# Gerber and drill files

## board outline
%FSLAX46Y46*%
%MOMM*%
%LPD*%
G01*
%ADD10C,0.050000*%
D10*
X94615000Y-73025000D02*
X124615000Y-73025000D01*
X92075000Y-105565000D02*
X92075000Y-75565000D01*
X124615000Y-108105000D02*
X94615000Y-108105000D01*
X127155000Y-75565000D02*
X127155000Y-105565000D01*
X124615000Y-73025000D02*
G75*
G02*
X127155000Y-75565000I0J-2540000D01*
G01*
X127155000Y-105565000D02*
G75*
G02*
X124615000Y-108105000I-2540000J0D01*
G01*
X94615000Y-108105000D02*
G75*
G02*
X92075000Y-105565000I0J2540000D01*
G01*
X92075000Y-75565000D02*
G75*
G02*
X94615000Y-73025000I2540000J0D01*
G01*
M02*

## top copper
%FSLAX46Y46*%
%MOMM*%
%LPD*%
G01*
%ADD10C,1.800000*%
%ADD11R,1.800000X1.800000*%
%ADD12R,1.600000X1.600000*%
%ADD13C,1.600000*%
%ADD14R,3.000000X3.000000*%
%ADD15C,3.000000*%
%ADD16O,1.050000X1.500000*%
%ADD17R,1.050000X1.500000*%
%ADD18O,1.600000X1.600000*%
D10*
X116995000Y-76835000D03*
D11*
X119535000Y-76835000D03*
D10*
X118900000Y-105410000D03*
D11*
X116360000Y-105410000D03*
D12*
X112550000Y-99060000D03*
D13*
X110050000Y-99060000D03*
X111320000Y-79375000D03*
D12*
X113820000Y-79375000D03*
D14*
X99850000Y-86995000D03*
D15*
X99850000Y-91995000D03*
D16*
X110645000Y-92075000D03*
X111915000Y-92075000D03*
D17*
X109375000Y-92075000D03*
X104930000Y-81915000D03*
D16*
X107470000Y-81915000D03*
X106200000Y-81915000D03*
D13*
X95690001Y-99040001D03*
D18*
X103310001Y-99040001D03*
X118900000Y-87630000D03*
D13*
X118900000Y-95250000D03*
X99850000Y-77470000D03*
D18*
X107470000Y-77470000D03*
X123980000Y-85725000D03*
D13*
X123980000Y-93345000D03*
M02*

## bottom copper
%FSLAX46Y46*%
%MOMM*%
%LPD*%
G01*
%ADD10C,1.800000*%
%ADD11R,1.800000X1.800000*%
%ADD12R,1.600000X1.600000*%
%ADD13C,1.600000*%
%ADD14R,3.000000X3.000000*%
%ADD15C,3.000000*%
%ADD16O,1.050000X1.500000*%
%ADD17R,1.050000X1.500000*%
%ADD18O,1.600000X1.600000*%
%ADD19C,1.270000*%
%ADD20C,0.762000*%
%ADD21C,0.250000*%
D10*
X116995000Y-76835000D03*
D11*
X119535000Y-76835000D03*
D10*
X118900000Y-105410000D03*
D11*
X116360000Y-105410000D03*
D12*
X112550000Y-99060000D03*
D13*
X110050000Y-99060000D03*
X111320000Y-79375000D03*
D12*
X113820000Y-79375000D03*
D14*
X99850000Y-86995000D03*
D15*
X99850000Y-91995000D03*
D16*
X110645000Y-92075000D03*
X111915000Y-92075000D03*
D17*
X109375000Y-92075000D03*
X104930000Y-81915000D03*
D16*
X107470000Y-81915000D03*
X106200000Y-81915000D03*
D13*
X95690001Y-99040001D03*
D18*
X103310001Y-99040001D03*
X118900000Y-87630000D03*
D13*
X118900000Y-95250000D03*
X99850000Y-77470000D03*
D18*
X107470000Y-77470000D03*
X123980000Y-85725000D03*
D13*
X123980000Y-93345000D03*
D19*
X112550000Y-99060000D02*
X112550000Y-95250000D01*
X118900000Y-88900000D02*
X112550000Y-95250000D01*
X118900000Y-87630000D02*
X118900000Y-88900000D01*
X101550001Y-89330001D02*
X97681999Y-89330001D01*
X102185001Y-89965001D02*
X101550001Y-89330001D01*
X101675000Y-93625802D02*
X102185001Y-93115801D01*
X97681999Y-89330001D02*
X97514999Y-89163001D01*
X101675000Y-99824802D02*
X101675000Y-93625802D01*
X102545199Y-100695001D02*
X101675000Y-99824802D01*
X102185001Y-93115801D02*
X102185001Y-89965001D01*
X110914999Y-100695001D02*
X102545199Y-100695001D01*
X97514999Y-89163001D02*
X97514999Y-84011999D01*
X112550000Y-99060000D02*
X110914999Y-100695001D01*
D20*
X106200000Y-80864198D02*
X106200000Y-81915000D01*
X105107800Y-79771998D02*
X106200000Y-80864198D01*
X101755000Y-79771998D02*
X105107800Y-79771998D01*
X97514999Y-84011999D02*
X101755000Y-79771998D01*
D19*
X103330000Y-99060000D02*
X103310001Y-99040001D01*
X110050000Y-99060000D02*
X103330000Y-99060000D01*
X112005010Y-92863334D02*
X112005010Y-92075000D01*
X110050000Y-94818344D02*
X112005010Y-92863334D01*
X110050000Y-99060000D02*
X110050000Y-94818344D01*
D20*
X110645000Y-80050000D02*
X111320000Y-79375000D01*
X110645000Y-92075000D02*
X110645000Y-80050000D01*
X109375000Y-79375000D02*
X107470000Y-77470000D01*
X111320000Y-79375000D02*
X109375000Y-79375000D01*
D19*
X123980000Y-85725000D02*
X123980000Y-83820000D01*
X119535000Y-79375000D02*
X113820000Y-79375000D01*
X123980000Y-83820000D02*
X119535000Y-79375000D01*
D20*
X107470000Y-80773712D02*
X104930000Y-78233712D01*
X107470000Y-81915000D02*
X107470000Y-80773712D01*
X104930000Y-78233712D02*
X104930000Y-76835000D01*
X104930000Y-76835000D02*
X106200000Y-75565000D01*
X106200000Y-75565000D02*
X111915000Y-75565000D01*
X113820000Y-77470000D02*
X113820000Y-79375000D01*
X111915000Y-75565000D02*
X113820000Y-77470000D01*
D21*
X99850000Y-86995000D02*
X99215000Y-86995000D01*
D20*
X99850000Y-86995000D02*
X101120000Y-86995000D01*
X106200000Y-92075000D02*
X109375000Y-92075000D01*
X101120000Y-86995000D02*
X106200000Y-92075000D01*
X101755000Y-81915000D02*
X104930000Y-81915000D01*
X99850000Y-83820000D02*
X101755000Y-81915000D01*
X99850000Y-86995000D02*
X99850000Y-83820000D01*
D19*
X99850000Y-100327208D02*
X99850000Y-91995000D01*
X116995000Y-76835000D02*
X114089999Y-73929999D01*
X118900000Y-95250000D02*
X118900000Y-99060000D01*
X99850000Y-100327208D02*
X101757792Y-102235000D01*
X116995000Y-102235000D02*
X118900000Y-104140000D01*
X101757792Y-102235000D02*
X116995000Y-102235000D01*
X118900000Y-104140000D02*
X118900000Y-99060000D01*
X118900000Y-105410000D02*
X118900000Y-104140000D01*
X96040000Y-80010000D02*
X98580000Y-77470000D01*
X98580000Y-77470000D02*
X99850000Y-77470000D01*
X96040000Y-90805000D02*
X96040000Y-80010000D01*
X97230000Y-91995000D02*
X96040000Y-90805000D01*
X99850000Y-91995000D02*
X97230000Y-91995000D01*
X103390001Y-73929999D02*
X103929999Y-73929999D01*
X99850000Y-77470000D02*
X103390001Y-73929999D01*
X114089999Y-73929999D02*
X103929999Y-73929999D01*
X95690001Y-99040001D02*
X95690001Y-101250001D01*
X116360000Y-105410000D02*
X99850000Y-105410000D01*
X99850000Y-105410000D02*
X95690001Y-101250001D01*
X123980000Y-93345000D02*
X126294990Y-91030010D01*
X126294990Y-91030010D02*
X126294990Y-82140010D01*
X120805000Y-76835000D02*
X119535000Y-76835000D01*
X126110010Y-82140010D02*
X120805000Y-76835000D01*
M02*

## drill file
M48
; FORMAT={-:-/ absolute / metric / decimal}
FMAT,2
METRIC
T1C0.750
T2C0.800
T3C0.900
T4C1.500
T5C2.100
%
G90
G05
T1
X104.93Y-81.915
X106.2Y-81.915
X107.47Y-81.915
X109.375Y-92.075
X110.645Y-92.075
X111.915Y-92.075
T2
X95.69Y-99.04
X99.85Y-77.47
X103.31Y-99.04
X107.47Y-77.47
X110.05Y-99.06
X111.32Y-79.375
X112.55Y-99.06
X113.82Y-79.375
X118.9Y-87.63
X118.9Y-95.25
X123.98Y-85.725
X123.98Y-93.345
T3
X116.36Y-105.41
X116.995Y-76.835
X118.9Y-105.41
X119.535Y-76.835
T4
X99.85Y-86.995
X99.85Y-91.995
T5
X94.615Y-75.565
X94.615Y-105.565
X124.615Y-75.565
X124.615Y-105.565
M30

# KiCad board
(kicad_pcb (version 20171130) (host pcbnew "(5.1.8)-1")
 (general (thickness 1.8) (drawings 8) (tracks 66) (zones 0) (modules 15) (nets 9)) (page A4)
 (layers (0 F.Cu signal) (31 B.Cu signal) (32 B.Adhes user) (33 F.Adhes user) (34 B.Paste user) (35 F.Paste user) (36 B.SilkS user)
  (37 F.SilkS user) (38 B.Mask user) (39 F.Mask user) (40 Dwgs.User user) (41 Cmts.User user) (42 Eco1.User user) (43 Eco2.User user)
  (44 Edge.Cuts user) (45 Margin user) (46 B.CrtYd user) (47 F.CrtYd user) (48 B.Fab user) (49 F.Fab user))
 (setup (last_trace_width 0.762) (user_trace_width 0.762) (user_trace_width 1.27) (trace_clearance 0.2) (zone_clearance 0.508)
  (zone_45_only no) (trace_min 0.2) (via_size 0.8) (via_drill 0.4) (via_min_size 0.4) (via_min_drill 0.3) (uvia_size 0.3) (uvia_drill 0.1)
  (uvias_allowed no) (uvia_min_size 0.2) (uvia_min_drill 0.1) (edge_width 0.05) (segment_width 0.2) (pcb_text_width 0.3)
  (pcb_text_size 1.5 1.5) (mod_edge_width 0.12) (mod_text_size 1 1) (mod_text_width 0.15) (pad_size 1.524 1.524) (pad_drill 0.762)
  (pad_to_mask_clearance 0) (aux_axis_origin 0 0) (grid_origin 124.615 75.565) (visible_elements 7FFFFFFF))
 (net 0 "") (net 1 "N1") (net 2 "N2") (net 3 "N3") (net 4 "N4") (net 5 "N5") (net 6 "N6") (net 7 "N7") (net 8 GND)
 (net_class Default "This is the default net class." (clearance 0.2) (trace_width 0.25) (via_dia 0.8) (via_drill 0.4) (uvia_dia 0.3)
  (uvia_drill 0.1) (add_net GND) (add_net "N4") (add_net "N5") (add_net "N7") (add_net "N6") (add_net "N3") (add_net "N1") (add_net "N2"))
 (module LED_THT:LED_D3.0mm (layer F.Cu) (at 119.535 76.835 180)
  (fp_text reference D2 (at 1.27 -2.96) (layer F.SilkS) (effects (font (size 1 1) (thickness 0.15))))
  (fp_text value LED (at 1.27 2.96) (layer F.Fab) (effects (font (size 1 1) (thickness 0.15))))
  (pad 2 thru_hole circle (at 2.54 0 180) (size 1.8 1.8) (drill 0.9) (layers *.Cu *.Mask) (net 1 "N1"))
  (pad 1 thru_hole rect (at 0 0 180) (size 1.8 1.8) (drill 0.9) (layers *.Cu *.Mask) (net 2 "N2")))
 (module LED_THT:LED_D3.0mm (layer F.Cu) (at 116.36 105.41)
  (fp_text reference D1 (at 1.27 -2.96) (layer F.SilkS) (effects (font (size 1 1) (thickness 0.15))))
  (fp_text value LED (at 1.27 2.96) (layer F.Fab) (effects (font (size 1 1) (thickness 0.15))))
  (pad 2 thru_hole circle (at 2.54 0) (size 1.8 1.8) (drill 0.9) (layers *.Cu *.Mask) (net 1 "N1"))
  (pad 1 thru_hole rect (at 0 0) (size 1.8 1.8) (drill 0.9) (layers *.Cu *.Mask) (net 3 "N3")))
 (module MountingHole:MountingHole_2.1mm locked (layer F.Cu) (at 124.615 105.565)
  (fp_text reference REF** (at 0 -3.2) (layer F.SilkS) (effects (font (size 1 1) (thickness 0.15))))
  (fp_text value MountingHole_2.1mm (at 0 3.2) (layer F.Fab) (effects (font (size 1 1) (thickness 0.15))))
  (pad "" np_thru_hole circle (at 0 0) (size 2.1 2.1) (drill 2.1) (layers *.Cu *.Mask)))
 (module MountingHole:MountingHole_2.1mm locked (layer F.Cu) (at 94.615 105.565)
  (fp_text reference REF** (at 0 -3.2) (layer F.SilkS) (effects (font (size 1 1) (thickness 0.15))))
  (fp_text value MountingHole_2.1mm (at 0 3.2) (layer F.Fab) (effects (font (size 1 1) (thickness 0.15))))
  (pad "" np_thru_hole circle (at 0 0) (size 2.1 2.1) (drill 2.1) (layers *.Cu *.Mask)))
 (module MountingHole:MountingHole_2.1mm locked (layer F.Cu) (at 124.615 75.565)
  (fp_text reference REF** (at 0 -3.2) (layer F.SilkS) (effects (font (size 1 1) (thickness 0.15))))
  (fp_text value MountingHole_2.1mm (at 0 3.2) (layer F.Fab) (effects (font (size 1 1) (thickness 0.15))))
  (pad "" np_thru_hole circle (at 0 0) (size 2.1 2.1) (drill 2.1) (layers *.Cu *.Mask)))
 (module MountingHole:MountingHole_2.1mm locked (layer F.Cu) (at 94.615 75.565)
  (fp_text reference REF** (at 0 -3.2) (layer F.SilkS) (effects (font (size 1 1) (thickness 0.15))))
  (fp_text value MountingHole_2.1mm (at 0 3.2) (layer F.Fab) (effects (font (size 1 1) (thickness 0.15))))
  (pad "" np_thru_hole circle (at 0 0) (size 2.1 2.1) (drill 2.1) (layers *.Cu *.Mask)))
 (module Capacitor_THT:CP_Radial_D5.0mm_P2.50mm (layer F.Cu) (at 112.55 99.06 180)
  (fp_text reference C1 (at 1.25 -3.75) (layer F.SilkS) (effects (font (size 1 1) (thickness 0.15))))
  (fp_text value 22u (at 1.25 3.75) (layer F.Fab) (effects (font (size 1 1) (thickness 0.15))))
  (pad 1 thru_hole rect (at 0 0 180) (size 1.6 1.6) (drill 0.8) (layers *.Cu *.Mask) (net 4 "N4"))
  (pad 2 thru_hole circle (at 2.5 0 180) (size 1.6 1.6) (drill 0.8) (layers *.Cu *.Mask) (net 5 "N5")))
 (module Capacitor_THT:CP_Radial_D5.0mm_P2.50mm (layer F.Cu) (at 113.82 79.375 180)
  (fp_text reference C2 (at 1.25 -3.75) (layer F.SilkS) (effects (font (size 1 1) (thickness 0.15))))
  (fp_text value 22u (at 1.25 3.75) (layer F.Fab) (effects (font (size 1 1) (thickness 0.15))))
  (pad 2 thru_hole circle (at 2.5 0 180) (size 1.6 1.6) (drill 0.8) (layers *.Cu *.Mask) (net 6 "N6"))
  (pad 1 thru_hole rect (at 0 0 180) (size 1.6 1.6) (drill 0.8) (layers *.Cu *.Mask) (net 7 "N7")))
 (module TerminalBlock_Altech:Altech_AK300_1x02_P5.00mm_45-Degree (layer F.Cu) (at 99.85 86.995 270)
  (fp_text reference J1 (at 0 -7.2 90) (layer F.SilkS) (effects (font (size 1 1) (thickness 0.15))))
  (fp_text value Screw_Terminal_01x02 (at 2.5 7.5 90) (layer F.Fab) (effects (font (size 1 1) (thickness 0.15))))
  (pad 1 thru_hole rect (at 0 0 270) (size 3 3) (drill 1.5) (layers *.Cu *.Mask) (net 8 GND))
  (pad 2 thru_hole circle (at 5 0 270) (size 3 3) (drill 1.5) (layers *.Cu *.Mask) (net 1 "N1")))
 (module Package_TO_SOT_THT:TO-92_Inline (layer F.Cu) (at 109.375 92.075)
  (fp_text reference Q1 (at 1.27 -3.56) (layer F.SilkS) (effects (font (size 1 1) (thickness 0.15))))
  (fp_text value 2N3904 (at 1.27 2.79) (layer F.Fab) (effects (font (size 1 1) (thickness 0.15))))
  (pad 2 thru_hole oval (at 1.27 0) (size 1.05 1.5) (drill 0.75) (layers *.Cu *.Mask) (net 6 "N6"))
  (pad 3 thru_hole oval (at 2.54 0) (size 1.05 1.5) (drill 0.75) (layers *.Cu *.Mask) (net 5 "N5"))
  (pad 1 thru_hole rect (at 0 0) (size 1.05 1.5) (drill 0.75) (layers *.Cu *.Mask) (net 8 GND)))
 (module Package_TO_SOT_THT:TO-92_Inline (layer F.Cu) (at 104.93 81.915)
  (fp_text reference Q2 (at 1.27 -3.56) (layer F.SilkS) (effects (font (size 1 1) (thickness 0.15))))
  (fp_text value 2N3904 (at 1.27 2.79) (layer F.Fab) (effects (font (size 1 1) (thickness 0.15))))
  (pad 1 thru_hole rect (at 0 0) (size 1.05 1.5) (drill 0.75) (layers *.Cu *.Mask) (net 8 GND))
  (pad 3 thru_hole oval (at 2.54 0) (size 1.05 1.5) (drill 0.75) (layers *.Cu *.Mask) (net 7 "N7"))
  (pad 2 thru_hole oval (at 1.27 0) (size 1.05 1.5) (drill 0.75) (layers *.Cu *.Mask) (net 4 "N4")))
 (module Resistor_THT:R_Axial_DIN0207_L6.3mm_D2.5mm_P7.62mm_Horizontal (layer F.Cu) (at 95.690001 99.040001)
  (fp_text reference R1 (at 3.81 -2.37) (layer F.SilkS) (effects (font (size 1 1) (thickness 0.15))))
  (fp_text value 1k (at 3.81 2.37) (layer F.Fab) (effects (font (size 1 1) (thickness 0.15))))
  (pad 1 thru_hole circle (at 0 0) (size 1.6 1.6) (drill 0.8) (layers *.Cu *.Mask) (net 3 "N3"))
  (pad 2 thru_hole oval (at 7.62 0) (size 1.6 1.6) (drill 0.8) (layers *.Cu *.Mask) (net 5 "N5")))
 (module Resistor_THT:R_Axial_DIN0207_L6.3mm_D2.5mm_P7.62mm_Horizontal (layer F.Cu) (at 118.9 95.25 90)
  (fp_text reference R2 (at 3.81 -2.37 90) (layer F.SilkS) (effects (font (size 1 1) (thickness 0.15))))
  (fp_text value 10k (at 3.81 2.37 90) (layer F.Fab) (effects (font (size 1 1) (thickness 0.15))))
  (pad 2 thru_hole oval (at 7.62 0 90) (size 1.6 1.6) (drill 0.8) (layers *.Cu *.Mask) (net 4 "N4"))
  (pad 1 thru_hole circle (at 0 0 90) (size 1.6 1.6) (drill 0.8) (layers *.Cu *.Mask) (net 1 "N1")))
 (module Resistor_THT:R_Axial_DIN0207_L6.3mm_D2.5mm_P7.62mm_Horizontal (layer F.Cu) (at 99.85 77.47)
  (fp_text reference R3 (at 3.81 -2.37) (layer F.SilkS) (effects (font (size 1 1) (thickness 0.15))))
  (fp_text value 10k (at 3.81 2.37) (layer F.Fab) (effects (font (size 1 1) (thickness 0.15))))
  (pad 1 thru_hole circle (at 0 0) (size 1.6 1.6) (drill 0.8) (layers *.Cu *.Mask) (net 1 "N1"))
  (pad 2 thru_hole oval (at 7.62 0) (size 1.6 1.6) (drill 0.8) (layers *.Cu *.Mask) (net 6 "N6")))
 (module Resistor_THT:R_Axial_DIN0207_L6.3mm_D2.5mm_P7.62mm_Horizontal (layer F.Cu) (at 123.98 93.345 90)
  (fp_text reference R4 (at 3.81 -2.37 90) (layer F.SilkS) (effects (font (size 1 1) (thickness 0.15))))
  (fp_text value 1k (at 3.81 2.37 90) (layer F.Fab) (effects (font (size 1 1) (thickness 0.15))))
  (pad 2 thru_hole oval (at 7.62 0 90) (size 1.6 1.6) (drill 0.8) (layers *.Cu *.Mask) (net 7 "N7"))
  (pad 1 thru_hole circle (at 0 0 90) (size 1.6 1.6) (drill 0.8) (layers *.Cu *.Mask) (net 2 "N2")))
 (gr_line (start 94.615 73.025) (end 124.615 73.025) (layer Edge.Cuts) (width 0.05))
 (gr_line (start 92.075 105.565) (end 92.075 75.565) (layer Edge.Cuts) (width 0.05))
 (gr_line (start 124.615 108.105) (end 94.615 108.105) (layer Edge.Cuts) (width 0.05))
 (gr_line (start 127.155 75.565) (end 127.155 105.565) (layer Edge.Cuts) (width 0.05))
 (gr_arc (start 124.615 75.565) (end 127.155 75.565) (angle -90) (layer Edge.Cuts) (width 0.05))
 (gr_arc (start 124.615 105.565) (end 124.615 108.105) (angle -90) (layer Edge.Cuts) (width 0.05))
 (gr_arc (start 94.615 105.565) (end 92.075 105.565) (angle -90) (layer Edge.Cuts) (width 0.05))
 (gr_arc (start 94.615 75.565) (end 94.615 73.025) (angle -90) (layer Edge.Cuts) (width 0.05))
 (segment (start 112.55 99.06) (end 112.55 95.25) (width 1.27) (layer B.Cu) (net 4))
 (segment (start 118.9 88.9) (end 112.55 95.25) (width 1.27) (layer B.Cu) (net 4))
 (segment (start 118.9 87.63) (end 118.9 88.9) (width 1.27) (layer B.Cu) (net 4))
 (segment (start 101.550001 89.330001) (end 97.681999 89.330001) (width 1.27) (layer B.Cu) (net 4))
 (segment (start 102.185001 89.965001) (end 101.550001 89.330001) (width 1.27) (layer B.Cu) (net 4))
 (segment (start 101.675 93.625802) (end 102.185001 93.115801) (width 1.27) (layer B.Cu) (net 4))
 (segment (start 97.681999 89.330001) (end 97.514999 89.163001) (width 1.27) (layer B.Cu) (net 4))
 (segment (start 101.675 99.824802) (end 101.675 93.625802) (width 1.27) (layer B.Cu) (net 4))
 (segment (start 102.545199 100.695001) (end 101.675 99.824802) (width 1.27) (layer B.Cu) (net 4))
 (segment (start 102.185001 93.115801) (end 102.185001 89.965001) (width 1.27) (layer B.Cu) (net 4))
 (segment (start 110.914999 100.695001) (end 102.545199 100.695001) (width 1.27) (layer B.Cu) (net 4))
 (segment (start 97.514999 89.163001) (end 97.514999 84.011999) (width 1.27) (layer B.Cu) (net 4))
 (segment (start 112.55 99.06) (end 110.914999 100.695001) (width 1.27) (layer B.Cu) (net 4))
 (segment (start 106.2 80.864198) (end 106.2 81.915) (width 0.762) (layer B.Cu) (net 4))
 (segment (start 105.1078 79.771998) (end 106.2 80.864198) (width 0.762) (layer B.Cu) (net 4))
 (segment (start 101.755 79.771998) (end 105.1078 79.771998) (width 0.762) (layer B.Cu) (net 4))
 (segment (start 97.514999 84.011999) (end 101.755 79.771998) (width 0.762) (layer B.Cu) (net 4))
 (segment (start 103.33 99.06) (end 103.310001 99.040001) (width 1.27) (layer B.Cu) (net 5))
 (segment (start 110.05 99.06) (end 103.33 99.06) (width 1.27) (layer B.Cu) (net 5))
 (segment (start 112.00501 92.863334) (end 112.00501 92.075) (width 1.27) (layer B.Cu) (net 5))
 (segment (start 110.05 94.818344) (end 112.00501 92.863334) (width 1.27) (layer B.Cu) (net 5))
 (segment (start 110.05 99.06) (end 110.05 94.818344) (width 1.27) (layer B.Cu) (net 5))
 (segment (start 110.645 80.05) (end 111.32 79.375) (width 0.762) (layer B.Cu) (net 6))
 (segment (start 110.645 92.075) (end 110.645 80.05) (width 0.762) (layer B.Cu) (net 6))
 (segment (start 109.375 79.375) (end 107.47 77.47) (width 0.762) (layer B.Cu) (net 6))
 (segment (start 111.32 79.375) (end 109.375 79.375) (width 0.762) (layer B.Cu) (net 6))
 (segment (start 123.98 85.725) (end 123.98 83.82) (width 1.27) (layer B.Cu) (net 7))
 (segment (start 119.535 79.375) (end 113.82 79.375) (width 1.27) (layer B.Cu) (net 7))
 (segment (start 123.98 83.82) (end 119.535 79.375) (width 1.27) (layer B.Cu) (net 7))
 (segment (start 107.47 80.773712) (end 104.93 78.233712) (width 0.762) (layer B.Cu) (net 7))
 (segment (start 107.47 81.915) (end 107.47 80.773712) (width 0.762) (layer B.Cu) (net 7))
 (segment (start 104.93 78.233712) (end 104.93 76.835) (width 0.762) (layer B.Cu) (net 7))
 (segment (start 104.93 76.835) (end 106.2 75.565) (width 0.762) (layer B.Cu) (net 7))
 (segment (start 106.2 75.565) (end 111.915 75.565) (width 0.762) (layer B.Cu) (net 7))
 (segment (start 113.82 77.47) (end 113.82 79.375) (width 0.762) (layer B.Cu) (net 7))
 (segment (start 111.915 75.565) (end 113.82 77.47) (width 0.762) (layer B.Cu) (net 7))
 (segment (start 99.85 86.995) (end 99.215 86.995) (width 0.25) (layer B.Cu) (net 8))
 (segment (start 99.85 86.995) (end 101.12 86.995) (width 0.762) (layer B.Cu) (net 8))
 (segment (start 106.2 92.075) (end 109.375 92.075) (width 0.762) (layer B.Cu) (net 8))
 (segment (start 101.12 86.995) (end 106.2 92.075) (width 0.762) (layer B.Cu) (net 8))
 (segment (start 101.755 81.915) (end 104.93 81.915) (width 0.762) (layer B.Cu) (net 8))
 (segment (start 99.85 83.82) (end 101.755 81.915) (width 0.762) (layer B.Cu) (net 8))
 (segment (start 99.85 86.995) (end 99.85 83.82) (width 0.762) (layer B.Cu) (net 8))
 (segment (start 99.85 100.327208) (end 99.85 91.995) (width 1.27) (layer B.Cu) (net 1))
 (segment (start 116.995 76.835) (end 114.089999 73.929999) (width 1.27) (layer B.Cu) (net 1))
 (segment (start 118.9 95.25) (end 118.9 99.06) (width 1.27) (layer B.Cu) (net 1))
 (segment (start 99.85 100.327208) (end 101.757792 102.235) (width 1.27) (layer B.Cu) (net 1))
 (segment (start 116.995 102.235) (end 118.9 104.14) (width 1.27) (layer B.Cu) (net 1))
 (segment (start 101.757792 102.235) (end 116.995 102.235) (width 1.27) (layer B.Cu) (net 1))
 (segment (start 118.9 104.14) (end 118.9 99.06) (width 1.27) (layer B.Cu) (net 1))
 (segment (start 118.9 105.41) (end 118.9 104.14) (width 1.27) (layer B.Cu) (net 1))
 (segment (start 96.04 80.01) (end 98.58 77.47) (width 1.27) (layer B.Cu) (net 1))
 (segment (start 98.58 77.47) (end 99.85 77.47) (width 1.27) (layer B.Cu) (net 1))
 (segment (start 96.04 90.805) (end 96.04 80.01) (width 1.27) (layer B.Cu) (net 1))
 (segment (start 97.23 91.995) (end 96.04 90.805) (width 1.27) (layer B.Cu) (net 1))
 (segment (start 99.85 91.995) (end 97.23 91.995) (width 1.27) (layer B.Cu) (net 1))
 (segment (start 103.390001 73.929999) (end 103.929999 73.929999) (width 1.27) (layer B.Cu) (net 1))
 (segment (start 99.85 77.47) (end 103.390001 73.929999) (width 1.27) (layer B.Cu) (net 1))
 (segment (start 114.089999 73.929999) (end 103.929999 73.929999) (width 1.27) (layer B.Cu) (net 1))
 (segment (start 95.690001 99.040001) (end 95.690001 101.250001) (width 1.27) (layer B.Cu) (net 3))
 (segment (start 116.36 105.41) (end 99.85 105.41) (width 1.27) (layer B.Cu) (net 3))
 (segment (start 99.85 105.41) (end 95.690001 101.250001) (width 1.27) (layer B.Cu) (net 3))
 (segment (start 123.98 93.345) (end 126.29499 91.03001) (width 1.27) (layer B.Cu) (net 2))
 (segment (start 126.29499 91.03001) (end 126.29499 82.14001) (width 1.27) (layer B.Cu) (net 2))
 (segment (start 120.805 76.835) (end 119.535 76.835) (width 1.27) (layer B.Cu) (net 2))
 (segment (start 126.11001 82.14001) (end 120.805 76.835) (width 1.27) (layer B.Cu) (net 2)))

